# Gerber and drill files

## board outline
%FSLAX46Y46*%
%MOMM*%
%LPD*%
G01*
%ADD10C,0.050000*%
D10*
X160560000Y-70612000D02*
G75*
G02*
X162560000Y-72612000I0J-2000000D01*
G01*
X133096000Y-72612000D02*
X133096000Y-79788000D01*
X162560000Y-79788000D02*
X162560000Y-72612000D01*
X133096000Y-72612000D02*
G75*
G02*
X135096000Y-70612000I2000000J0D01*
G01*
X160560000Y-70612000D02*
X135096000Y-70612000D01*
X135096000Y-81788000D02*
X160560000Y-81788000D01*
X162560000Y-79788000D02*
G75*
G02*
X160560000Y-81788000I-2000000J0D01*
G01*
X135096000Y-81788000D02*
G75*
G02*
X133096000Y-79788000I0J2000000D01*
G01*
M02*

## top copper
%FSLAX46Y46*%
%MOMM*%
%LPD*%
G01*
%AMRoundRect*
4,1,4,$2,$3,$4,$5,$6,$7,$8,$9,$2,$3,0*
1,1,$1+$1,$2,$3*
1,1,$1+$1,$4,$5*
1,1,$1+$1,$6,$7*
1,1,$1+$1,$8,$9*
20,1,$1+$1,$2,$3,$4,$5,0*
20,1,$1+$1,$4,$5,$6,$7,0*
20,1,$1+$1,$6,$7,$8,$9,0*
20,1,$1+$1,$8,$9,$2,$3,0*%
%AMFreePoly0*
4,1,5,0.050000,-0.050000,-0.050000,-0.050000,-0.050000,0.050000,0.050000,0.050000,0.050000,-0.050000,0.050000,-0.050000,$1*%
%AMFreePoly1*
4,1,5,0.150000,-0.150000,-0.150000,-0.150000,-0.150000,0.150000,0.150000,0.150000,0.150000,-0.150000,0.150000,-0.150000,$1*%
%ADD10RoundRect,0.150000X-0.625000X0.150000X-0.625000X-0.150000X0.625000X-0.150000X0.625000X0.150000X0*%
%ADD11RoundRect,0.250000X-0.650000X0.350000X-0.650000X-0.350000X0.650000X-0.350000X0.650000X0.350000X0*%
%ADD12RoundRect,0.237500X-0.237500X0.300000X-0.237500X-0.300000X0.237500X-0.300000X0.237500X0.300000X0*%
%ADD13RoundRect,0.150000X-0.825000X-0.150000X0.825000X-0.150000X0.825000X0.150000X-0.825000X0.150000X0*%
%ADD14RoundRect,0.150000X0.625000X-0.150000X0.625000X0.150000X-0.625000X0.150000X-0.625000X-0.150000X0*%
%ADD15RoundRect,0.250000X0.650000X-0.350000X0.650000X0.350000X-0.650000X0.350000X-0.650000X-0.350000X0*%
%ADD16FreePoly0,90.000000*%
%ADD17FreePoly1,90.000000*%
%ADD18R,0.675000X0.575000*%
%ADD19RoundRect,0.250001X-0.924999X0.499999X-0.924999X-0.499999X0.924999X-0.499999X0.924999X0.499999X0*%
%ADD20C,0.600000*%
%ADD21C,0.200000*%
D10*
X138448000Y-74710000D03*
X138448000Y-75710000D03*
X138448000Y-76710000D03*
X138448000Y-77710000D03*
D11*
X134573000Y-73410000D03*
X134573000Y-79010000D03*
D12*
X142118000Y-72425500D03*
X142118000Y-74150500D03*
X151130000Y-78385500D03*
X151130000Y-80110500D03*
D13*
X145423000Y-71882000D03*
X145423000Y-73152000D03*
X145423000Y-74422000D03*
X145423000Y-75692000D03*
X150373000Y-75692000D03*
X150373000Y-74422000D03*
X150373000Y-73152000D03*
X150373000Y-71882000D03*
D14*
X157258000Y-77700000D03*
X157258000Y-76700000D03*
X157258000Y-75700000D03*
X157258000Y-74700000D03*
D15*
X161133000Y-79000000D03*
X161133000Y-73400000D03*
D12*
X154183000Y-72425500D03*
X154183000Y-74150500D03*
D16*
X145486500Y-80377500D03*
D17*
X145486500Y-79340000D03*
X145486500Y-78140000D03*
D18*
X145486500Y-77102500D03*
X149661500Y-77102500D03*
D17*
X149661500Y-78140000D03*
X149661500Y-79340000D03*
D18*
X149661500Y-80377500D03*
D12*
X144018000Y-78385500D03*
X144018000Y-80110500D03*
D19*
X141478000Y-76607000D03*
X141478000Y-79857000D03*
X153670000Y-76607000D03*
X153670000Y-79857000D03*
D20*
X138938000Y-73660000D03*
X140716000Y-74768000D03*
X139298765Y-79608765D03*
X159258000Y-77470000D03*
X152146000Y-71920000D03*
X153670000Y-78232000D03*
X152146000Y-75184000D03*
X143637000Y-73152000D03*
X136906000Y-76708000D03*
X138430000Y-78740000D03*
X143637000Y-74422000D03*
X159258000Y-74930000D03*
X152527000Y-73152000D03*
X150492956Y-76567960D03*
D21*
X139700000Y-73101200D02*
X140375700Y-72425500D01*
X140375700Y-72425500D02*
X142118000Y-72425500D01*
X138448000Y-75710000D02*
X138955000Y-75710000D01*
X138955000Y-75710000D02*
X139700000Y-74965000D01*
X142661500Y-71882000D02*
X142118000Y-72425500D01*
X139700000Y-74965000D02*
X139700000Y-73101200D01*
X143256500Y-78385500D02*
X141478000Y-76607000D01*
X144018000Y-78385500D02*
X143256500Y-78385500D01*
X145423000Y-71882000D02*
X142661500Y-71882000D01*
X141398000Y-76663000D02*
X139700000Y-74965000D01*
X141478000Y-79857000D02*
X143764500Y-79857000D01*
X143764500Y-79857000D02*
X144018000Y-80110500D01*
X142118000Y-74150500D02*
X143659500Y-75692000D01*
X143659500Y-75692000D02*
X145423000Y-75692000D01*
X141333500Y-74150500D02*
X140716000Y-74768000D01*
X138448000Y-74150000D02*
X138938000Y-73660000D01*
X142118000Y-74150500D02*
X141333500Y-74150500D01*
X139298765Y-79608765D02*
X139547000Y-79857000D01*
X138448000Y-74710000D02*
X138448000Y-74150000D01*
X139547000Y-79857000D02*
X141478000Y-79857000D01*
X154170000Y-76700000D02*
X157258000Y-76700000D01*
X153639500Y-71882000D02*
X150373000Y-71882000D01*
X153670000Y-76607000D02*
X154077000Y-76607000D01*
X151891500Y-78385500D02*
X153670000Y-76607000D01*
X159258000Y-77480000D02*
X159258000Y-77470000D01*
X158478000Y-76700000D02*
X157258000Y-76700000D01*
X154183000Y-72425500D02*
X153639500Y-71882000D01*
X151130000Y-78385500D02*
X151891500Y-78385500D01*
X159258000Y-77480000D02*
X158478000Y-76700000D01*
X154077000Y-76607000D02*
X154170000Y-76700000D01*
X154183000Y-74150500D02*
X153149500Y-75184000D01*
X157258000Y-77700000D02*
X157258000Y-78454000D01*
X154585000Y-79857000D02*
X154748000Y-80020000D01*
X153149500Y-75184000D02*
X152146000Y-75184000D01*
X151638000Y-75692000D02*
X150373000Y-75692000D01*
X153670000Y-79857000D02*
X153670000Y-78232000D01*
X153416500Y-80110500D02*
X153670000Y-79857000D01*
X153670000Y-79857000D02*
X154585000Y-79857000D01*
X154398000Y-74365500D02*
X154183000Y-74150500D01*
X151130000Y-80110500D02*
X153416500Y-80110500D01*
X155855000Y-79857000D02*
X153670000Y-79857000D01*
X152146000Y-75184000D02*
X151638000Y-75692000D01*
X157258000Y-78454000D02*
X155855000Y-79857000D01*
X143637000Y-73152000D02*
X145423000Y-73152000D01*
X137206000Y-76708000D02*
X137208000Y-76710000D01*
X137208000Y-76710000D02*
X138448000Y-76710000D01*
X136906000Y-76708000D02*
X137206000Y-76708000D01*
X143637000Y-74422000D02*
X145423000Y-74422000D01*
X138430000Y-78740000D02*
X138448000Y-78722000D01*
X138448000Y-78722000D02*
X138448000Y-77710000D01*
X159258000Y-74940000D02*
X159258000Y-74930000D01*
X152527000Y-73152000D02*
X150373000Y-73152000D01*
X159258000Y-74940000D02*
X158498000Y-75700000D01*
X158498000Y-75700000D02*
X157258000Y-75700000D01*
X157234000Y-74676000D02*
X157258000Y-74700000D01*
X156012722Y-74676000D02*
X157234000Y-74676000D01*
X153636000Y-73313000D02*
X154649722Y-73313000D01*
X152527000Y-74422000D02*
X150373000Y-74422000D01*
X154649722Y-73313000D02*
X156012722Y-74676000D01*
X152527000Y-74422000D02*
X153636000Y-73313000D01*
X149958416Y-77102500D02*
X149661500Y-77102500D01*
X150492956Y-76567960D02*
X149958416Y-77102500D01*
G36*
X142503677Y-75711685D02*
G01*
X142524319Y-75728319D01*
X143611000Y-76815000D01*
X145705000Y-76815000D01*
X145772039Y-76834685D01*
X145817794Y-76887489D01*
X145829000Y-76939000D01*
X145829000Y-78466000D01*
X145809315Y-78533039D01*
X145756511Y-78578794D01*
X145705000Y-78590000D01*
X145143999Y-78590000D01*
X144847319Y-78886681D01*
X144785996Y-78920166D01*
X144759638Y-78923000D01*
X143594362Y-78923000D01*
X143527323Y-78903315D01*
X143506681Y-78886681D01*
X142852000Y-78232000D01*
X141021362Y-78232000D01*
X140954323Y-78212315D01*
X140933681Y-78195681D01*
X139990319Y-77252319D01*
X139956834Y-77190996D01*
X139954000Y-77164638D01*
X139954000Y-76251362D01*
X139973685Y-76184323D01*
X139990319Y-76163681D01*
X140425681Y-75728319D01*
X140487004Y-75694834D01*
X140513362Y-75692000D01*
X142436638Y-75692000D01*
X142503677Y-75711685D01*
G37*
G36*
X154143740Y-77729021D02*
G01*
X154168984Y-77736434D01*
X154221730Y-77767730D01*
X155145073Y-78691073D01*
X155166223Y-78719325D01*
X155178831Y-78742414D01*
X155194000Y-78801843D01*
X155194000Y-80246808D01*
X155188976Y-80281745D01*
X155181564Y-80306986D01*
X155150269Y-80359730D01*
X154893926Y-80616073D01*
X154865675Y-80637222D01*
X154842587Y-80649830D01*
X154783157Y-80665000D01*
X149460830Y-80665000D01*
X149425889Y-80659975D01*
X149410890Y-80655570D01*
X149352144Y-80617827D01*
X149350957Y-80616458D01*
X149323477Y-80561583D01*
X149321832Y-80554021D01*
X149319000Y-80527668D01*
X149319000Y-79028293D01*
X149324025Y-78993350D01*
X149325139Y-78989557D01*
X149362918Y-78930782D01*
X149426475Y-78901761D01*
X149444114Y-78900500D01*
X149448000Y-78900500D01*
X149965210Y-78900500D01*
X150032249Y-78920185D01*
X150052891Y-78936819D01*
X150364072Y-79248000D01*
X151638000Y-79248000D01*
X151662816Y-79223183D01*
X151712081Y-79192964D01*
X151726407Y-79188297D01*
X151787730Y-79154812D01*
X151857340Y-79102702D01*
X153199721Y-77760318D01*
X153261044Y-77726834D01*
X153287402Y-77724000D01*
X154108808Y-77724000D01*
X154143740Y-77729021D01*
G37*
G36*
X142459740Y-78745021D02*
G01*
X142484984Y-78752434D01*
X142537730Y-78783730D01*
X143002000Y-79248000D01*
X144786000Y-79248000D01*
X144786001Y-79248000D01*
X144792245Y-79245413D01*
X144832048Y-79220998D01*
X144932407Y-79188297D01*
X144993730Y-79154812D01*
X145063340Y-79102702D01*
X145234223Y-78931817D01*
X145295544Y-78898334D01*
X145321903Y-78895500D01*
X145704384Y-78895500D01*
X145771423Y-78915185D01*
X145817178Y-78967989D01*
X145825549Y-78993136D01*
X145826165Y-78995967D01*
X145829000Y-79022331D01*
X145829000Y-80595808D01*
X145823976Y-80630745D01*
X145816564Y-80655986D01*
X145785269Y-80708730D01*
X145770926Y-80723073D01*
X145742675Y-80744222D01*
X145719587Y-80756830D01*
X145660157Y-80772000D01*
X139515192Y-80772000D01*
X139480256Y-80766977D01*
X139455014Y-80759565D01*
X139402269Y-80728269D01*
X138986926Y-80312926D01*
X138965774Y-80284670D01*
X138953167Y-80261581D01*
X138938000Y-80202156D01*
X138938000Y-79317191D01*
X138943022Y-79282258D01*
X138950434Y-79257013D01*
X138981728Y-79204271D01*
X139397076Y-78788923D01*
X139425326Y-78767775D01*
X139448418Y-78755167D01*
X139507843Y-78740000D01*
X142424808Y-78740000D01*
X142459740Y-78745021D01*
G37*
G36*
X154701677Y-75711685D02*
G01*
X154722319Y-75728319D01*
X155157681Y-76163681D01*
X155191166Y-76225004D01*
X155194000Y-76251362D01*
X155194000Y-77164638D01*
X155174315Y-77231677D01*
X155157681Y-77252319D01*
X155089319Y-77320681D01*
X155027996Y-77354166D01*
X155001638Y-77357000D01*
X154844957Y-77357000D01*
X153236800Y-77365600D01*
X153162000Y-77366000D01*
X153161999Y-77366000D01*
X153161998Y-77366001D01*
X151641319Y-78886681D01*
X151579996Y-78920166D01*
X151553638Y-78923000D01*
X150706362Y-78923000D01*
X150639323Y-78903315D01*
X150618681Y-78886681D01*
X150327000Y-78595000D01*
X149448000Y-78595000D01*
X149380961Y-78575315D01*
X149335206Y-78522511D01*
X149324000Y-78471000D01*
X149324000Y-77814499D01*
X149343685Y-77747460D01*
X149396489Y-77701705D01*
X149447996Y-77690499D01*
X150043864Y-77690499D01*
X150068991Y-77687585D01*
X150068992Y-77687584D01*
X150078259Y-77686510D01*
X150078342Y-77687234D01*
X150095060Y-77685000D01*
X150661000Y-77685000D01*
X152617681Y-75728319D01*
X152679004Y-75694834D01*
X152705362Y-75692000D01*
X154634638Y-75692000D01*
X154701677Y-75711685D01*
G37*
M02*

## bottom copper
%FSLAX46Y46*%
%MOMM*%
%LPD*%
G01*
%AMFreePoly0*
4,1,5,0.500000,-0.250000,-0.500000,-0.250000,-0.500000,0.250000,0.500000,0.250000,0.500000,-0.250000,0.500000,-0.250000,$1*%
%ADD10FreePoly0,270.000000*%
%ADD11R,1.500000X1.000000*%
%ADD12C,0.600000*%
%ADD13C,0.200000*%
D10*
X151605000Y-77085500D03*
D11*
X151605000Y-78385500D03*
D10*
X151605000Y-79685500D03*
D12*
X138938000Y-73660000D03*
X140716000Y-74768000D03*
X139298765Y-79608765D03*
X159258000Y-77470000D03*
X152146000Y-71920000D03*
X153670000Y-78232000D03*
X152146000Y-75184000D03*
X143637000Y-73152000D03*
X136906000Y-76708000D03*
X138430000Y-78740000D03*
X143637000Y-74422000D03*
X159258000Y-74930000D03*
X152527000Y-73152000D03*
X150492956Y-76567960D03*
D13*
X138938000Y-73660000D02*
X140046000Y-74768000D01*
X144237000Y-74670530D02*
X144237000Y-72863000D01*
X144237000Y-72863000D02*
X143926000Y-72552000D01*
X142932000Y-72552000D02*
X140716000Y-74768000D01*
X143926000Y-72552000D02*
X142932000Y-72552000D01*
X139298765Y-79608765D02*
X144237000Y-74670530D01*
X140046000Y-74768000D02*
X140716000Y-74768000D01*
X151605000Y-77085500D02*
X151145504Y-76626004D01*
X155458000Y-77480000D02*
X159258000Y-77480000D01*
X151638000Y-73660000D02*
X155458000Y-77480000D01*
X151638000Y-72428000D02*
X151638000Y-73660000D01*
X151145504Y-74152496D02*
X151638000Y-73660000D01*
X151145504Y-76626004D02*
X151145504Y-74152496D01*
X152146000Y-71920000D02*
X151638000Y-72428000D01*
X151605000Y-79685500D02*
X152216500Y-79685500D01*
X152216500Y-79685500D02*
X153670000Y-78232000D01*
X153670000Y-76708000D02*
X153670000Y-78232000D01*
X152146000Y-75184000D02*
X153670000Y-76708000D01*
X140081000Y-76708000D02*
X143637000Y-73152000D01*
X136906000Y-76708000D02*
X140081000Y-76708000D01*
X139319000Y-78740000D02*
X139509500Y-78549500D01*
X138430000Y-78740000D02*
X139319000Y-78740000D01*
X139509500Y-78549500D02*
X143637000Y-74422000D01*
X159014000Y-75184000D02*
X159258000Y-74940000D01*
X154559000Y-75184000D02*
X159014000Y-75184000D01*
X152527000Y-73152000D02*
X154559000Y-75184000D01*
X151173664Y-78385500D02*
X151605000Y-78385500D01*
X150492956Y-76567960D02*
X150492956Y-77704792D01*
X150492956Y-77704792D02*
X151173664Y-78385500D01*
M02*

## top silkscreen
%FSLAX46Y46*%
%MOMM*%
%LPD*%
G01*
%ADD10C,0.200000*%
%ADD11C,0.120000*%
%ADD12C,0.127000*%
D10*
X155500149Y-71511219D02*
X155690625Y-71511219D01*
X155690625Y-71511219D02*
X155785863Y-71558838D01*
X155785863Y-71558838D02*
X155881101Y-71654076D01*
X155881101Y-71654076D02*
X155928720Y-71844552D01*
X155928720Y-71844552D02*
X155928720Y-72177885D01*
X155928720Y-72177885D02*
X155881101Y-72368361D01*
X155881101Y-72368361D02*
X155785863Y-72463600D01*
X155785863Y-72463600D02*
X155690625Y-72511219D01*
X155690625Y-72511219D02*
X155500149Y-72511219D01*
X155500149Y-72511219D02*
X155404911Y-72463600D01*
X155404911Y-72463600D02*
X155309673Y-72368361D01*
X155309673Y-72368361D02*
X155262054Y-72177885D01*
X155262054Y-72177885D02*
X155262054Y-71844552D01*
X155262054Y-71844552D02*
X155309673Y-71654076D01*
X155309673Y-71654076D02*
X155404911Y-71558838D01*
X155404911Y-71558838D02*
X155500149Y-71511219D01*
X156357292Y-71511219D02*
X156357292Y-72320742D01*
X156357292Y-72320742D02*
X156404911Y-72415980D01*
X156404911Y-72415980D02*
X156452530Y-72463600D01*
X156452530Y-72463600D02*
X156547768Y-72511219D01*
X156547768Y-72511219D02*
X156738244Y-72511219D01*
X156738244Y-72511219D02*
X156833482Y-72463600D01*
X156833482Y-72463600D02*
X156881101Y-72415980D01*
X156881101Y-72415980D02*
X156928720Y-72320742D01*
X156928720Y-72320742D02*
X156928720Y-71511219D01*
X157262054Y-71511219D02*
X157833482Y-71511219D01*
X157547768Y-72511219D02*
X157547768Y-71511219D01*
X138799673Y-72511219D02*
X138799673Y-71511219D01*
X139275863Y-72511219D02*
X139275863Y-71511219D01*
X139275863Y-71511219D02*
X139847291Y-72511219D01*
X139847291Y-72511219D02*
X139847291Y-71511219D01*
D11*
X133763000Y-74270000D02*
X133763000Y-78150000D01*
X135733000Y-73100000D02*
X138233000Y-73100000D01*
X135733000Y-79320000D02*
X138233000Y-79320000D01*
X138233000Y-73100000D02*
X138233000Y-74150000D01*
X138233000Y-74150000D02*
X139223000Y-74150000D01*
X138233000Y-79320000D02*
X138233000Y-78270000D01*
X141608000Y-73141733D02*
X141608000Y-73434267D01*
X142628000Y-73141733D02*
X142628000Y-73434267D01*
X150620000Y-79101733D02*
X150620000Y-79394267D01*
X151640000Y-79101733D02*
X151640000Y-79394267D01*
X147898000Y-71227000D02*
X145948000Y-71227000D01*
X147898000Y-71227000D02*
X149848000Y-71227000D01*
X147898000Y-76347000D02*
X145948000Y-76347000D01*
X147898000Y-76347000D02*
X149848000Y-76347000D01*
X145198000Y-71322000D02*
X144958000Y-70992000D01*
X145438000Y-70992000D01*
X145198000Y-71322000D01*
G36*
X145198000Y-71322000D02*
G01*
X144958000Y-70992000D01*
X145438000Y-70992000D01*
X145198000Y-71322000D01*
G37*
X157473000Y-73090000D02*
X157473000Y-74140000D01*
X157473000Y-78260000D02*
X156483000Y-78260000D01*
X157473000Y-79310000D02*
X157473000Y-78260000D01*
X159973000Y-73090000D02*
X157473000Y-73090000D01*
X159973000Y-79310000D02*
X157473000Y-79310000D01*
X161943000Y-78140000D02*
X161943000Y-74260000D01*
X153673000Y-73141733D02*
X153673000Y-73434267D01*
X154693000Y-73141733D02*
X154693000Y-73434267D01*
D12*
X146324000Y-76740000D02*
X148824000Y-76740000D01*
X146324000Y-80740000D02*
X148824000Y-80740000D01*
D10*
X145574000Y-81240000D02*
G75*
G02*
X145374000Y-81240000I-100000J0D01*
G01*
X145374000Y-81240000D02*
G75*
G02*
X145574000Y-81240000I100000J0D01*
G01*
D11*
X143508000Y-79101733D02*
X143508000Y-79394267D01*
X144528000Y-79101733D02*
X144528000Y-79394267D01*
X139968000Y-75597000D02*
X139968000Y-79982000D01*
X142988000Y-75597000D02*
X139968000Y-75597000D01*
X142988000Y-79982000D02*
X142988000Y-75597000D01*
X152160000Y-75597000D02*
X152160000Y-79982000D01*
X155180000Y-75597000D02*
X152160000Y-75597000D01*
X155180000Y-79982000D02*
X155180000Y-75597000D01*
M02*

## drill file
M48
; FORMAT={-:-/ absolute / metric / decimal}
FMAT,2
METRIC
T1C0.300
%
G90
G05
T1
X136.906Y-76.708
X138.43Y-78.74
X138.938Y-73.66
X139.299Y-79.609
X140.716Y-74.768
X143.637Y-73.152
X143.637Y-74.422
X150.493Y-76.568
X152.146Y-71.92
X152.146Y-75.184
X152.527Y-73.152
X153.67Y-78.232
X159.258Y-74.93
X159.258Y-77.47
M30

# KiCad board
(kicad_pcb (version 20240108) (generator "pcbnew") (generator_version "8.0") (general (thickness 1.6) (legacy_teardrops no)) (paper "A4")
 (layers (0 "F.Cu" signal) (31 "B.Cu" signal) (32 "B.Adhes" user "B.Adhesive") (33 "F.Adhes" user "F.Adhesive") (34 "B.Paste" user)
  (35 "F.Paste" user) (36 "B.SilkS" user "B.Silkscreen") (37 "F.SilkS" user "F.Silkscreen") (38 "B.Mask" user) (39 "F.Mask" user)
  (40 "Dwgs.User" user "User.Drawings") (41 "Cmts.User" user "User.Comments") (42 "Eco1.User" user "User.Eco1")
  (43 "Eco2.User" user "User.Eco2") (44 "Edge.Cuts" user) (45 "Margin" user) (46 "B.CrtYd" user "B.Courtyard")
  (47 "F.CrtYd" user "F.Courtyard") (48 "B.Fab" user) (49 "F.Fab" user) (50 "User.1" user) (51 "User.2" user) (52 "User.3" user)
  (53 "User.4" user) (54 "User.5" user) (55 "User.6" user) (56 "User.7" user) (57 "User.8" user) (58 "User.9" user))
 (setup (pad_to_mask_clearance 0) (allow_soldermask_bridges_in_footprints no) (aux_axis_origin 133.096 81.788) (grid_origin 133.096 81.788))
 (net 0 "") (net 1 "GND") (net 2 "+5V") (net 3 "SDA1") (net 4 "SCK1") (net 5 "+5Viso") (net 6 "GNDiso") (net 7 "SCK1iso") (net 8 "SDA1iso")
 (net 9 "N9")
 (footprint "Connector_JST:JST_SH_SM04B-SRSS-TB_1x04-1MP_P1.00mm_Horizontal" (layer "F.Cu") (at 136.448 76.21 -90)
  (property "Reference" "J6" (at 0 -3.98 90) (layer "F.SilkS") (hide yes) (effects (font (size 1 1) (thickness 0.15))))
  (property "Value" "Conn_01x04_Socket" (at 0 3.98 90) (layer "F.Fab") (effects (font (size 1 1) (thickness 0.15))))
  (fp_line (start -1.94 2.685) (end 1.94 2.685) (stroke (width 0.12) (type solid)) (layer "F.SilkS"))
  (fp_line (start -3.11 0.715) (end -3.11 -1.785) (stroke (width 0.12) (type solid)) (layer "F.SilkS"))
  (fp_line (start 3.11 0.715) (end 3.11 -1.785) (stroke (width 0.12) (type solid)) (layer "F.SilkS"))
  (fp_line (start -3.11 -1.785) (end -2.06 -1.785) (stroke (width 0.12) (type solid)) (layer "F.SilkS"))
  (fp_line (start -2.06 -1.785) (end -2.06 -2.775) (stroke (width 0.12) (type solid)) (layer "F.SilkS"))
  (fp_line (start 3.11 -1.785) (end 2.06 -1.785) (stroke (width 0.12) (type solid)) (layer "F.SilkS"))
  (pad "1" smd roundrect (at -1.5 -2 270) (size 0.6 1.55) (layers "F.Cu" "F.Paste" "F.Mask") (roundrect_rratio 0.25) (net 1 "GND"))
  (pad "2" smd roundrect (at -0.5 -2 270) (size 0.6 1.55) (layers "F.Cu" "F.Paste" "F.Mask") (roundrect_rratio 0.25) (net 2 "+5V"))
  (pad "3" smd roundrect (at 0.5 -2 270) (size 0.6 1.55) (layers "F.Cu" "F.Paste" "F.Mask") (roundrect_rratio 0.25) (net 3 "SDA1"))
  (pad "4" smd roundrect (at 1.5 -2 270) (size 0.6 1.55) (layers "F.Cu" "F.Paste" "F.Mask") (roundrect_rratio 0.25) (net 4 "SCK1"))
  (pad "MP" smd roundrect (at -2.8 1.875 270) (size 1.2 1.8) (layers "F.Cu" "F.Paste" "F.Mask") (roundrect_rratio 0.208333))
  (pad "MP" smd roundrect (at 2.8 1.875 270) (size 1.2 1.8) (layers "F.Cu" "F.Paste" "F.Mask") (roundrect_rratio 0.208333)))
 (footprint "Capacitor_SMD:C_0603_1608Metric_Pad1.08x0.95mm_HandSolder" (layer "F.Cu") (at 142.118 73.288 -90)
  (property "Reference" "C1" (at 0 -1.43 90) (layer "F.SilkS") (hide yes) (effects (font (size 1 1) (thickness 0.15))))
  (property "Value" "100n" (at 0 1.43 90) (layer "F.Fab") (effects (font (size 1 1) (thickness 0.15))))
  (fp_line (start -0.146267 0.51) (end 0.146267 0.51) (stroke (width 0.12) (type solid)) (layer "F.SilkS"))
  (fp_line (start -0.146267 -0.51) (end 0.146267 -0.51) (stroke (width 0.12) (type solid)) (layer "F.SilkS"))
  (pad "1" smd roundrect (at -0.8625 0 270) (size 1.075 0.95) (layers "F.Cu" "F.Paste" "F.Mask") (roundrect_rratio 0.25) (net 2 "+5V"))
  (pad "2" smd roundrect (at 0.8625 0 270) (size 1.075 0.95) (layers "F.Cu" "F.Paste" "F.Mask") (roundrect_rratio 0.25) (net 1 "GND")))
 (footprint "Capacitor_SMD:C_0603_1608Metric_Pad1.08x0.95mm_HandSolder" (layer "F.Cu") (at 151.13 79.248 -90)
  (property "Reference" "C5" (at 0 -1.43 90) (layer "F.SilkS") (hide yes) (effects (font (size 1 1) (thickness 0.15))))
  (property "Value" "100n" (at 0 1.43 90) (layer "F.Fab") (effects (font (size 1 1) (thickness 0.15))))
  (fp_line (start -0.146267 0.51) (end 0.146267 0.51) (stroke (width 0.12) (type solid)) (layer "F.SilkS"))
  (fp_line (start -0.146267 -0.51) (end 0.146267 -0.51) (stroke (width 0.12) (type solid)) (layer "F.SilkS"))
  (pad "1" smd roundrect (at -0.8625 0 270) (size 1.075 0.95) (layers "F.Cu" "F.Paste" "F.Mask") (roundrect_rratio 0.25) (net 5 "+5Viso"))
  (pad "2" smd roundrect (at 0.8625 0 270) (size 1.075 0.95) (layers "F.Cu" "F.Paste" "F.Mask") (roundrect_rratio 0.25) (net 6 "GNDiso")))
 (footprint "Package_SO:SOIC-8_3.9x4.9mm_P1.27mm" (layer "F.Cu") (at 147.898 73.787)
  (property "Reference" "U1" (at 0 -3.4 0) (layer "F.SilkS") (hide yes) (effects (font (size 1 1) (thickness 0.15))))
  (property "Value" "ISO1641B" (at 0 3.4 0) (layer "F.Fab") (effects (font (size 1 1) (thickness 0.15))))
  (fp_line (start 0 -2.56) (end -1.95 -2.56) (stroke (width 0.12) (type solid)) (layer "F.SilkS"))
  (fp_line (start 0 -2.56) (end 1.95 -2.56) (stroke (width 0.12) (type solid)) (layer "F.SilkS"))
  (fp_line (start 0 2.56) (end -1.95 2.56) (stroke (width 0.12) (type solid)) (layer "F.SilkS"))
  (fp_line (start 0 2.56) (end 1.95 2.56) (stroke (width 0.12) (type solid)) (layer "F.SilkS"))
  (fp_poly
   (pts (xy -2.7 -2.465) (xy -2.94 -2.795) (xy -2.46 -2.795) (xy -2.7 -2.465)) (stroke (width 0.12) (type solid)) (fill solid)
   (layer "F.SilkS"))
  (pad "1" smd roundrect (at -2.475 -1.905) (size 1.95 0.6) (layers "F.Cu" "F.Paste" "F.Mask") (roundrect_rratio 0.25) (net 2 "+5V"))
  (pad "2" smd roundrect (at -2.475 -0.635) (size 1.95 0.6) (layers "F.Cu" "F.Paste" "F.Mask") (roundrect_rratio 0.25) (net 3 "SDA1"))
  (pad "3" smd roundrect (at -2.475 0.635) (size 1.95 0.6) (layers "F.Cu" "F.Paste" "F.Mask") (roundrect_rratio 0.25) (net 4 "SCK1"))
  (pad "4" smd roundrect (at -2.475 1.905) (size 1.95 0.6) (layers "F.Cu" "F.Paste" "F.Mask") (roundrect_rratio 0.25) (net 1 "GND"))
  (pad "5" smd roundrect (at 2.475 1.905) (size 1.95 0.6) (layers "F.Cu" "F.Paste" "F.Mask") (roundrect_rratio 0.25) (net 6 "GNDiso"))
  (pad "6" smd roundrect (at 2.475 0.635) (size 1.95 0.6) (layers "F.Cu" "F.Paste" "F.Mask") (roundrect_rratio 0.25) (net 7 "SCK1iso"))
  (pad "7" smd roundrect (at 2.475 -0.635) (size 1.95 0.6) (layers "F.Cu" "F.Paste" "F.Mask") (roundrect_rratio 0.25) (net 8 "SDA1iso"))
  (pad "8" smd roundrect (at 2.475 -1.905) (size 1.95 0.6) (layers "F.Cu" "F.Paste" "F.Mask") (roundrect_rratio 0.25) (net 5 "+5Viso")))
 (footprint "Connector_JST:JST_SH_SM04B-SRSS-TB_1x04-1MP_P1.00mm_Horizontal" (layer "F.Cu") (at 159.258 76.2 90)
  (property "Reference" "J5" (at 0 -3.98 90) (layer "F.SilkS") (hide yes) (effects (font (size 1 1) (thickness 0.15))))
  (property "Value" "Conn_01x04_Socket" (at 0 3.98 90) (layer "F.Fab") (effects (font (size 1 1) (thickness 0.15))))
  (fp_line (start 3.11 -1.785) (end 2.06 -1.785) (stroke (width 0.12) (type solid)) (layer "F.SilkS"))
  (fp_line (start -2.06 -1.785) (end -2.06 -2.775) (stroke (width 0.12) (type solid)) (layer "F.SilkS"))
  (fp_line (start -3.11 -1.785) (end -2.06 -1.785) (stroke (width 0.12) (type solid)) (layer "F.SilkS"))
  (fp_line (start 3.11 0.715) (end 3.11 -1.785) (stroke (width 0.12) (type solid)) (layer "F.SilkS"))
  (fp_line (start -3.11 0.715) (end -3.11 -1.785) (stroke (width 0.12) (type solid)) (layer "F.SilkS"))
  (fp_line (start -1.94 2.685) (end 1.94 2.685) (stroke (width 0.12) (type solid)) (layer "F.SilkS"))
  (pad "1" smd roundrect (at -1.5 -2 90) (size 0.6 1.55) (layers "F.Cu" "F.Paste" "F.Mask") (roundrect_rratio 0.25) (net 6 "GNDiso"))
  (pad "2" smd roundrect (at -0.5 -2 90) (size 0.6 1.55) (layers "F.Cu" "F.Paste" "F.Mask") (roundrect_rratio 0.25) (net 5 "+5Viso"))
  (pad "3" smd roundrect (at 0.5 -2 90) (size 0.6 1.55) (layers "F.Cu" "F.Paste" "F.Mask") (roundrect_rratio 0.25) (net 8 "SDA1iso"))
  (pad "4" smd roundrect (at 1.5 -2 90) (size 0.6 1.55) (layers "F.Cu" "F.Paste" "F.Mask") (roundrect_rratio 0.25) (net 7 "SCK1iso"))
  (pad "MP" smd roundrect (at -2.8 1.875 90) (size 1.2 1.8) (layers "F.Cu" "F.Paste" "F.Mask") (roundrect_rratio 0.208333))
  (pad "MP" smd roundrect (at 2.8 1.875 90) (size 1.2 1.8) (layers "F.Cu" "F.Paste" "F.Mask") (roundrect_rratio 0.208333)))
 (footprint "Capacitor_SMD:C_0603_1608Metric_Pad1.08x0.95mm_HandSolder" (layer "F.Cu") (at 154.183 73.288 -90)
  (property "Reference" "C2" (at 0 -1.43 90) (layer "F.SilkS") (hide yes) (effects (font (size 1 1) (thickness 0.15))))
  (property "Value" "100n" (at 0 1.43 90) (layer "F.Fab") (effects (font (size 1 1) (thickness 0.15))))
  (fp_line (start -0.146267 0.51) (end 0.146267 0.51) (stroke (width 0.12) (type solid)) (layer "F.SilkS"))
  (fp_line (start -0.146267 -0.51) (end 0.146267 -0.51) (stroke (width 0.12) (type solid)) (layer "F.SilkS"))
  (pad "1" smd roundrect (at -0.8625 0 270) (size 1.075 0.95) (layers "F.Cu" "F.Paste" "F.Mask") (roundrect_rratio 0.25) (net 5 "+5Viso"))
  (pad "2" smd roundrect (at 0.8625 0 270) (size 1.075 0.95) (layers "F.Cu" "F.Paste" "F.Mask") (roundrect_rratio 0.25) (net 6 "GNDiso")))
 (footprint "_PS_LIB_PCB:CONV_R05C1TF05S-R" (layer "F.Cu") (at 147.574 78.74 90)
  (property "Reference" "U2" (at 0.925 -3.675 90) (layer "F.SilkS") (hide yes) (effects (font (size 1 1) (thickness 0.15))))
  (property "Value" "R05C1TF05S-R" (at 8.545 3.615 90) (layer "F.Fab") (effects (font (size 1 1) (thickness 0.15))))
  (fp_line (start 2 -1.25) (end 2 1.25) (stroke (width 0.127) (type solid)) (layer "F.SilkS"))
  (fp_line (start -2 -1.25) (end -2 1.25) (stroke (width 0.127) (type solid)) (layer "F.SilkS"))
  (fp_circle (center -2.5 -2.1) (end -2.4 -2.1) (stroke (width 0.2) (type solid)) (fill none) (layer "F.SilkS"))
  (pad "1" smd custom (at -1.6375 -2.0875 90) (size 0.1 0.1) (layers "F.Cu") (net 1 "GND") (options (clearance outline) (anchor rect))
   (primitives))
  (pad "2_3" smd custom (at -0.6 -2.0875 90) (size 0.3 0.3) (layers "F.Cu") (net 1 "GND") (options (clearance outline) (anchor rect))
   (primitives))
  (pad "4_5" smd custom (at 0.6 -2.0875 90) (size 0.3 0.3) (layers "F.Cu") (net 2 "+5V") (options (clearance outline) (anchor rect))
   (primitives))
  (pad "6" smd rect (at 1.6375 -2.0875 90) (size 0.575 0.675) (layers "F.Cu" "F.Paste" "F.Mask") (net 2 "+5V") (solder_mask_margin 0.102))
  (pad "7" smd rect (at 1.6375 2.0875 90) (size 0.575 0.675) (layers "F.Cu" "F.Paste" "F.Mask") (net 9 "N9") (solder_mask_margin 0.102))
  (pad "8_9" smd custom (at 0.6 2.0875 90) (size 0.3 0.3) (layers "F.Cu") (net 5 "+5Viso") (options (clearance outline) (anchor rect))
   (primitives))
  (pad "10_11" smd custom (at -0.6 2.0875 90) (size 0.3 0.3) (layers "F.Cu") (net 6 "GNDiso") (options (clearance outline) (anchor rect))
   (primitives))
  (pad "12" smd rect (at -1.6375 2.0875 90) (size 0.575 0.675) (layers "F.Cu" "F.Paste" "F.Mask") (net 6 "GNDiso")
   (solder_mask_margin 0.102)))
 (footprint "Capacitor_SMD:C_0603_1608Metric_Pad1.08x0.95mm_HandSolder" (layer "F.Cu") (at 144.018 79.248 -90)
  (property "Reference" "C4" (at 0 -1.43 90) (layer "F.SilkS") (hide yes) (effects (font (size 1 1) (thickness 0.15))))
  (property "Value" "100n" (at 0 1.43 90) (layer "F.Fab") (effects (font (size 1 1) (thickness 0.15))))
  (fp_line (start -0.146267 0.51) (end 0.146267 0.51) (stroke (width 0.12) (type solid)) (layer "F.SilkS"))
  (fp_line (start -0.146267 -0.51) (end 0.146267 -0.51) (stroke (width 0.12) (type solid)) (layer "F.SilkS"))
  (pad "1" smd roundrect (at -0.8625 0 270) (size 1.075 0.95) (layers "F.Cu" "F.Paste" "F.Mask") (roundrect_rratio 0.25) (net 2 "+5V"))
  (pad "2" smd roundrect (at 0.8625 0 270) (size 1.075 0.95) (layers "F.Cu" "F.Paste" "F.Mask") (roundrect_rratio 0.25) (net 1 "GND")))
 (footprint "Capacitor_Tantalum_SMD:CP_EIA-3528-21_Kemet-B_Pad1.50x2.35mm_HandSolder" (layer "F.Cu") (at 141.478 78.232 -90)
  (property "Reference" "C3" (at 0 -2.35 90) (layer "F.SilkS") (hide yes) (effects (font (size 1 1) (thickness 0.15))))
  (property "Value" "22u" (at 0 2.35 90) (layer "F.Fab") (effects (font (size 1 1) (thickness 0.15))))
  (fp_line (start -2.635 1.51) (end 1.75 1.51) (stroke (width 0.12) (type solid)) (layer "F.SilkS"))
  (fp_line (start -2.635 -1.51) (end -2.635 1.51) (stroke (width 0.12) (type solid)) (layer "F.SilkS"))
  (fp_line (start 1.75 -1.51) (end -2.635 -1.51) (stroke (width 0.12) (type solid)) (layer "F.SilkS"))
  (pad "1" smd roundrect (at -1.625 0 270) (size 1.5 2.35) (layers "F.Cu" "F.Paste" "F.Mask") (roundrect_rratio 0.166667) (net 2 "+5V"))
  (pad "2" smd roundrect (at 1.625 0 270) (size 1.5 2.35) (layers "F.Cu" "F.Paste" "F.Mask") (roundrect_rratio 0.166667) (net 1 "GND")))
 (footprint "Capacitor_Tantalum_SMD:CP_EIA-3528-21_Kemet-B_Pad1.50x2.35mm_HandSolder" (layer "F.Cu") (at 153.67 78.232 -90)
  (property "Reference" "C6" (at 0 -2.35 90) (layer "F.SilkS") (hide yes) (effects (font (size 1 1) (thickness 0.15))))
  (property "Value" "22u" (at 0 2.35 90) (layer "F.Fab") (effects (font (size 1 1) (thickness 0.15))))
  (fp_line (start -2.635 1.51) (end 1.75 1.51) (stroke (width 0.12) (type solid)) (layer "F.SilkS"))
  (fp_line (start -2.635 -1.51) (end -2.635 1.51) (stroke (width 0.12) (type solid)) (layer "F.SilkS"))
  (fp_line (start 1.75 -1.51) (end -2.635 -1.51) (stroke (width 0.12) (type solid)) (layer "F.SilkS"))
  (pad "1" smd roundrect (at -1.625 0 270) (size 1.5 2.35) (layers "F.Cu" "F.Paste" "F.Mask") (roundrect_rratio 0.166667) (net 5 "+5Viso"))
  (pad "2" smd roundrect (at 1.625 0 270) (size 1.5 2.35) (layers "F.Cu" "F.Paste" "F.Mask") (roundrect_rratio 0.166667) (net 6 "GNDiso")))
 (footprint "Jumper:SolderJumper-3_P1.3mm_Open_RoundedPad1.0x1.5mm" (layer "B.Cu") (at 151.605 78.3855 -90)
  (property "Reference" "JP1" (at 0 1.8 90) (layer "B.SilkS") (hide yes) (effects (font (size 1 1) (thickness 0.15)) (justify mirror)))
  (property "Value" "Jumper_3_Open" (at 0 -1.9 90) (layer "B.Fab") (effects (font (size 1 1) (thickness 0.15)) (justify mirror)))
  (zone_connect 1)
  (pad "1" smd custom (at -1.3 0 270) (size 1 0.5) (layers "B.Cu" "B.Mask") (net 5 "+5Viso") (zone_connect 2) (thermal_bridge_angle 45)
   (options (clearance outline) (anchor rect)) (primitives))
  (pad "2" smd rect (at 0 0 270) (size 1 1.5) (layers "B.Cu" "B.Mask") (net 9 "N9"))
  (pad "3" smd custom (at 1.3 0 270) (size 1 0.5) (layers "B.Cu" "B.Mask") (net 6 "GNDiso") (zone_connect 2) (thermal_bridge_angle 45)
   (options (clearance outline) (anchor rect)) (primitives)))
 (gr_arc (start 160.56 70.612) (mid 161.974214 71.197786) (end 162.56 72.612) (stroke (width 0.05) (type default)) (layer "Edge.Cuts"))
 (gr_line (start 133.096 72.612) (end 133.096 79.788) (stroke (width 0.05) (type default)) (layer "Edge.Cuts"))
 (gr_line (start 162.56 79.788) (end 162.56 72.612) (stroke (width 0.05) (type default)) (layer "Edge.Cuts"))
 (gr_arc (start 133.096 72.612) (mid 133.681786 71.197786) (end 135.096 70.612) (stroke (width 0.05) (type default)) (layer "Edge.Cuts"))
 (gr_line (start 160.56 70.612) (end 135.096 70.612) (stroke (width 0.05) (type default)) (layer "Edge.Cuts"))
 (gr_line (start 135.096 81.788) (end 160.56 81.788) (stroke (width 0.05) (type default)) (layer "Edge.Cuts"))
 (gr_arc (start 162.56 79.788) (mid 161.974214 81.202214) (end 160.56 81.788) (stroke (width 0.05) (type default)) (layer "Edge.Cuts"))
 (gr_arc (start 135.096 81.788) (mid 133.681786 81.202214) (end 133.096 79.788) (stroke (width 0.05) (type default)) (layer "Edge.Cuts"))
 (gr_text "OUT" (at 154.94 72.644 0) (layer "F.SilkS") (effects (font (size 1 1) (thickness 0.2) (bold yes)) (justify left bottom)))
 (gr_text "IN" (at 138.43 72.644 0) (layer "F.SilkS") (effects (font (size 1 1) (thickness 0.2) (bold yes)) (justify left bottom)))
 (segment (start 139.7 73.1012) (end 140.3757 72.4255) (width 0.2) (layer "F.Cu") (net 2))
 (segment (start 140.3757 72.4255) (end 142.118 72.4255) (width 0.2) (layer "F.Cu") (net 2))
 (segment (start 138.448 75.71) (end 138.955 75.71) (width 0.2) (layer "F.Cu") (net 2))
 (segment (start 138.955 75.71) (end 139.7 74.965) (width 0.2) (layer "F.Cu") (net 2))
 (segment (start 142.6615 71.882) (end 142.118 72.4255) (width 0.2) (layer "F.Cu") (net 2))
 (segment (start 139.7 74.965) (end 139.7 73.1012) (width 0.2) (layer "F.Cu") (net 2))
 (segment (start 143.2565 78.3855) (end 141.478 76.607) (width 0.2) (layer "F.Cu") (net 2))
 (segment (start 144.018 78.3855) (end 143.2565 78.3855) (width 0.2) (layer "F.Cu") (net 2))
 (segment (start 145.423 71.882) (end 142.6615 71.882) (width 0.2) (layer "F.Cu") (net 2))
 (segment (start 141.398 76.663) (end 139.7 74.965) (width 0.2) (layer "F.Cu") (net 2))
 (segment (start 141.478 79.857) (end 143.7645 79.857) (width 0.2) (layer "F.Cu") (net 1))
 (segment (start 143.7645 79.857) (end 144.018 80.1105) (width 0.2) (layer "F.Cu") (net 1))
 (segment (start 142.118 74.1505) (end 143.6595 75.692) (width 0.2) (layer "F.Cu") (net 1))
 (segment (start 143.6595 75.692) (end 145.423 75.692) (width 0.2) (layer "F.Cu") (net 1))
 (segment (start 141.3335 74.1505) (end 140.716 74.768) (width 0.2) (layer "F.Cu") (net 1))
 (segment (start 138.448 74.15) (end 138.938 73.66) (width 0.2) (layer "F.Cu") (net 1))
 (segment (start 142.118 74.1505) (end 141.3335 74.1505) (width 0.2) (layer "F.Cu") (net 1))
 (segment (start 139.298765 79.608765) (end 139.547 79.857) (width 0.2) (layer "F.Cu") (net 1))
 (segment (start 138.448 74.71) (end 138.448 74.15) (width 0.2) (layer "F.Cu") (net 1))
 (segment (start 139.547 79.857) (end 141.478 79.857) (width 0.2) (layer "F.Cu") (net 1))
 (via (at 138.938 73.66) (size 0.6) (drill 0.3) (layers "F.Cu" "B.Cu") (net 1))
 (via (at 140.716 74.768) (size 0.6) (drill 0.3) (layers "F.Cu" "B.Cu") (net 1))
 (via (at 139.298765 79.608765) (size 0.6) (drill 0.3) (layers "F.Cu" "B.Cu") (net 1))
 (segment (start 138.938 73.66) (end 140.046 74.768) (width 0.2) (layer "B.Cu") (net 1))
 (segment (start 144.237 74.67053) (end 144.237 72.863) (width 0.2) (layer "B.Cu") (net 1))
 (segment (start 144.237 72.863) (end 143.926 72.552) (width 0.2) (layer "B.Cu") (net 1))
 (segment (start 142.932 72.552) (end 140.716 74.768) (width 0.2) (layer "B.Cu") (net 1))
 (segment (start 143.926 72.552) (end 142.932 72.552) (width 0.2) (layer "B.Cu") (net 1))
 (segment (start 139.298765 79.608765) (end 144.237 74.67053) (width 0.2) (layer "B.Cu") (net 1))
 (segment (start 140.046 74.768) (end 140.716 74.768) (width 0.2) (layer "B.Cu") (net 1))
 (segment (start 154.17 76.7) (end 157.258 76.7) (width 0.2) (layer "F.Cu") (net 5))
 (segment (start 153.6395 71.882) (end 150.373 71.882) (width 0.2) (layer "F.Cu") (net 5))
 (segment (start 153.67 76.607) (end 154.077 76.607) (width 0.2) (layer "F.Cu") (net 5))
 (segment (start 151.8915 78.3855) (end 153.67 76.607) (width 0.2) (layer "F.Cu") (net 5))
 (segment (start 159.258 77.48) (end 159.258 77.47) (width 0.2) (layer "F.Cu") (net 5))
 (segment (start 158.478 76.7) (end 157.258 76.7) (width 0.2) (layer "F.Cu") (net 5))
 (segment (start 154.183 72.4255) (end 153.6395 71.882) (width 0.2) (layer "F.Cu") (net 5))
 (segment (start 151.13 78.3855) (end 151.8915 78.3855) (width 0.2) (layer "F.Cu") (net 5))
 (segment (start 159.258 77.48) (end 158.478 76.7) (width 0.2) (layer "F.Cu") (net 5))
 (segment (start 154.077 76.607) (end 154.17 76.7) (width 0.2) (layer "F.Cu") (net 5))
 (via (at 159.258 77.47) (size 0.6) (drill 0.3) (layers "F.Cu" "B.Cu") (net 5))
 (via (at 152.146 71.92) (size 0.6) (drill 0.3) (layers "F.Cu" "B.Cu") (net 5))
 (segment (start 151.605 77.0855) (end 151.145504 76.626004) (width 0.2) (layer "B.Cu") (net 5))
 (segment (start 155.458 77.48) (end 159.258 77.48) (width 0.2) (layer "B.Cu") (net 5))
 (segment (start 151.638 73.66) (end 155.458 77.48) (width 0.2) (layer "B.Cu") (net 5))
 (segment (start 151.638 72.428) (end 151.638 73.66) (width 0.2) (layer "B.Cu") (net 5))
 (segment (start 151.145504 74.152496) (end 151.638 73.66) (width 0.2) (layer "B.Cu") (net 5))
 (segment (start 151.145504 76.626004) (end 151.145504 74.152496) (width 0.2) (layer "B.Cu") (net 5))
 (segment (start 152.146 71.92) (end 151.638 72.428) (width 0.2) (layer "B.Cu") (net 5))
 (segment (start 154.183 74.1505) (end 153.1495 75.184) (width 0.2) (layer "F.Cu") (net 6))
 (segment (start 157.258 77.7) (end 157.258 78.454) (width 0.2) (layer "F.Cu") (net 6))
 (segment (start 154.585 79.857) (end 154.748 80.02) (width 0.2) (layer "F.Cu") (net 6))
 (segment (start 153.1495 75.184) (end 152.146 75.184) (width 0.2) (layer "F.Cu") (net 6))
 (segment (start 151.638 75.692) (end 150.373 75.692) (width 0.2) (layer "F.Cu") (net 6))
 (segment (start 153.67 79.857) (end 153.67 78.232) (width 0.2) (layer "F.Cu") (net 6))
 (segment (start 153.4165 80.1105) (end 153.67 79.857) (width 0.2) (layer "F.Cu") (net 6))
 (segment (start 153.67 79.857) (end 154.585 79.857) (width 0.2) (layer "F.Cu") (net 6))
 (segment (start 154.398 74.3655) (end 154.183 74.1505) (width 0.2) (layer "F.Cu") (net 6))
 (segment (start 151.13 80.1105) (end 153.4165 80.1105) (width 0.2) (layer "F.Cu") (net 6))
 (segment (start 155.855 79.857) (end 153.67 79.857) (width 0.2) (layer "F.Cu") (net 6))
 (segment (start 152.146 75.184) (end 151.638 75.692) (width 0.2) (layer "F.Cu") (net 6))
 (segment (start 157.258 78.454) (end 155.855 79.857) (width 0.2) (layer "F.Cu") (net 6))
 (via (at 153.67 78.232) (size 0.6) (drill 0.3) (layers "F.Cu" "B.Cu") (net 6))
 (via (at 152.146 75.184) (size 0.6) (drill 0.3) (layers "F.Cu" "B.Cu") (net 6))
 (segment (start 151.605 79.6855) (end 152.2165 79.6855) (width 0.2) (layer "B.Cu") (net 6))
 (segment (start 152.2165 79.6855) (end 153.67 78.232) (width 0.2) (layer "B.Cu") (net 6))
 (segment (start 153.67 76.708) (end 153.67 78.232) (width 0.2) (layer "B.Cu") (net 6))
 (segment (start 152.146 75.184) (end 153.67 76.708) (width 0.2) (layer "B.Cu") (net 6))
 (segment (start 143.637 73.152) (end 145.423 73.152) (width 0.2) (layer "F.Cu") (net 3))
 (segment (start 137.206 76.708) (end 137.208 76.71) (width 0.2) (layer "F.Cu") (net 3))
 (segment (start 137.208 76.71) (end 138.448 76.71) (width 0.2) (layer "F.Cu") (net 3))
 (segment (start 136.906 76.708) (end 137.206 76.708) (width 0.2) (layer "F.Cu") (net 3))
 (via (at 143.637 73.152) (size 0.6) (drill 0.3) (layers "F.Cu" "B.Cu") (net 3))
 (via (at 136.906 76.708) (size 0.6) (drill 0.3) (layers "F.Cu" "B.Cu") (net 3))
 (segment (start 140.081 76.708) (end 143.637 73.152) (width 0.2) (layer "B.Cu") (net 3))
 (segment (start 136.906 76.708) (end 140.081 76.708) (width 0.2) (layer "B.Cu") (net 3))
 (segment (start 143.637 74.422) (end 145.423 74.422) (width 0.2) (layer "F.Cu") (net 4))
 (segment (start 138.43 78.74) (end 138.448 78.722) (width 0.2) (layer "F.Cu") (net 4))
 (segment (start 138.448 78.722) (end 138.448 77.71) (width 0.2) (layer "F.Cu") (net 4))
 (via (at 138.43 78.74) (size 0.6) (drill 0.3) (layers "F.Cu" "B.Cu") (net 4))
 (via (at 143.637 74.422) (size 0.6) (drill 0.3) (layers "F.Cu" "B.Cu") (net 4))
 (segment (start 139.319 78.74) (end 139.5095 78.5495) (width 0.2) (layer "B.Cu") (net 4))
 (segment (start 138.43 78.74) (end 139.319 78.74) (width 0.2) (layer "B.Cu") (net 4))
 (segment (start 139.5095 78.5495) (end 143.637 74.422) (width 0.2) (layer "B.Cu") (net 4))
 (segment (start 159.258 74.94) (end 159.258 74.93) (width 0.2) (layer "F.Cu") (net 8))
 (segment (start 152.527 73.152) (end 150.373 73.152) (width 0.2) (layer "F.Cu") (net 8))
 (segment (start 159.258 74.94) (end 158.498 75.7) (width 0.2) (layer "F.Cu") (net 8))
 (segment (start 158.498 75.7) (end 157.258 75.7) (width 0.2) (layer "F.Cu") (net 8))
 (via (at 159.258 74.93) (size 0.6) (drill 0.3) (layers "F.Cu" "B.Cu") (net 8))
 (via (at 152.527 73.152) (size 0.6) (drill 0.3) (layers "F.Cu" "B.Cu") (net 8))
 (segment (start 159.014 75.184) (end 159.258 74.94) (width 0.2) (layer "B.Cu") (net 8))
 (segment (start 154.559 75.184) (end 159.014 75.184) (width 0.2) (layer "B.Cu") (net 8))
 (segment (start 152.527 73.152) (end 154.559 75.184) (width 0.2) (layer "B.Cu") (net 8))
 (segment (start 157.234 74.676) (end 157.258 74.7) (width 0.2) (layer "F.Cu") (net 7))
 (segment (start 156.012722 74.676) (end 157.234 74.676) (width 0.2) (layer "F.Cu") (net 7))
 (segment (start 153.636 73.313) (end 154.649722 73.313) (width 0.2) (layer "F.Cu") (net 7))
 (segment (start 152.527 74.422) (end 150.373 74.422) (width 0.2) (layer "F.Cu") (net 7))
 (segment (start 154.649722 73.313) (end 156.012722 74.676) (width 0.2) (layer "F.Cu") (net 7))
 (segment (start 152.527 74.422) (end 153.636 73.313) (width 0.2) (layer "F.Cu") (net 7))
 (segment (start 149.958416 77.1025) (end 149.6615 77.1025) (width 0.2) (layer "F.Cu") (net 9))
 (segment (start 150.492956 76.56796) (end 149.958416 77.1025) (width 0.2) (layer "F.Cu") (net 9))
 (via (at 150.492956 76.56796) (size 0.6) (drill 0.3) (layers "F.Cu" "B.Cu") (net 9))
 (segment (start 151.173664 78.3855) (end 151.605 78.3855) (width 0.2) (layer "B.Cu") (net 9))
 (segment (start 150.492956 76.56796) (end 150.492956 77.704792) (width 0.2) (layer "B.Cu") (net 9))
 (segment (start 150.492956 77.704792) (end 151.173664 78.3855) (width 0.2) (layer "B.Cu") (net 9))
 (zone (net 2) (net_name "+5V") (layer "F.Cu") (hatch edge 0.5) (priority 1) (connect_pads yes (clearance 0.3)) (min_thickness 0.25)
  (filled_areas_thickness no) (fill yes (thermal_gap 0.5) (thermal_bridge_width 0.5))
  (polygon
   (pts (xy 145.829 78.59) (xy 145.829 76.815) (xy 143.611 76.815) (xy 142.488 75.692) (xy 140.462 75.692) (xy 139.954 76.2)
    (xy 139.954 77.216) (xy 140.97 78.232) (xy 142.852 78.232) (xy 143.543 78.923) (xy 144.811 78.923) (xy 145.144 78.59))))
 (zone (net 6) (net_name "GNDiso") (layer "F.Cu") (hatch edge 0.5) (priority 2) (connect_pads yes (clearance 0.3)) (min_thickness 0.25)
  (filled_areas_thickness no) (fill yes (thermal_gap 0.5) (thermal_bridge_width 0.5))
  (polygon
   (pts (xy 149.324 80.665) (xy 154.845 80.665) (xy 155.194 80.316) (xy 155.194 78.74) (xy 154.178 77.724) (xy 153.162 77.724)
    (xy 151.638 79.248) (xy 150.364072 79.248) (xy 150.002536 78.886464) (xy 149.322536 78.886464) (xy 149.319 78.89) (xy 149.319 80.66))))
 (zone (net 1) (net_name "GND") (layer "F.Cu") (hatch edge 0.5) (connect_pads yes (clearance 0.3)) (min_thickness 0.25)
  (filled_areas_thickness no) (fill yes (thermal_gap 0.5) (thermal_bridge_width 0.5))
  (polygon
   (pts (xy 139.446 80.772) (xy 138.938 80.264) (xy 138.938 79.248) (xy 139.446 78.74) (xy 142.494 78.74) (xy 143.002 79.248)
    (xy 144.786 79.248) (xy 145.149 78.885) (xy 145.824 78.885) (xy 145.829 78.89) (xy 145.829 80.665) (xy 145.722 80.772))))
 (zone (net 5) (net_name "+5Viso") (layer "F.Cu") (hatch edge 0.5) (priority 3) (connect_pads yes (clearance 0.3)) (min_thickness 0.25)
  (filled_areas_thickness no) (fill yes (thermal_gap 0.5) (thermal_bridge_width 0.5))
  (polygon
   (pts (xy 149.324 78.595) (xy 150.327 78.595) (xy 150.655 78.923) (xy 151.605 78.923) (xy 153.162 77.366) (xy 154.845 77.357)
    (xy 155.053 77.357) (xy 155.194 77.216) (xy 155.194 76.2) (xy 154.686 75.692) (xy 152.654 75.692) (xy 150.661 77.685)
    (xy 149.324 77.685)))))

